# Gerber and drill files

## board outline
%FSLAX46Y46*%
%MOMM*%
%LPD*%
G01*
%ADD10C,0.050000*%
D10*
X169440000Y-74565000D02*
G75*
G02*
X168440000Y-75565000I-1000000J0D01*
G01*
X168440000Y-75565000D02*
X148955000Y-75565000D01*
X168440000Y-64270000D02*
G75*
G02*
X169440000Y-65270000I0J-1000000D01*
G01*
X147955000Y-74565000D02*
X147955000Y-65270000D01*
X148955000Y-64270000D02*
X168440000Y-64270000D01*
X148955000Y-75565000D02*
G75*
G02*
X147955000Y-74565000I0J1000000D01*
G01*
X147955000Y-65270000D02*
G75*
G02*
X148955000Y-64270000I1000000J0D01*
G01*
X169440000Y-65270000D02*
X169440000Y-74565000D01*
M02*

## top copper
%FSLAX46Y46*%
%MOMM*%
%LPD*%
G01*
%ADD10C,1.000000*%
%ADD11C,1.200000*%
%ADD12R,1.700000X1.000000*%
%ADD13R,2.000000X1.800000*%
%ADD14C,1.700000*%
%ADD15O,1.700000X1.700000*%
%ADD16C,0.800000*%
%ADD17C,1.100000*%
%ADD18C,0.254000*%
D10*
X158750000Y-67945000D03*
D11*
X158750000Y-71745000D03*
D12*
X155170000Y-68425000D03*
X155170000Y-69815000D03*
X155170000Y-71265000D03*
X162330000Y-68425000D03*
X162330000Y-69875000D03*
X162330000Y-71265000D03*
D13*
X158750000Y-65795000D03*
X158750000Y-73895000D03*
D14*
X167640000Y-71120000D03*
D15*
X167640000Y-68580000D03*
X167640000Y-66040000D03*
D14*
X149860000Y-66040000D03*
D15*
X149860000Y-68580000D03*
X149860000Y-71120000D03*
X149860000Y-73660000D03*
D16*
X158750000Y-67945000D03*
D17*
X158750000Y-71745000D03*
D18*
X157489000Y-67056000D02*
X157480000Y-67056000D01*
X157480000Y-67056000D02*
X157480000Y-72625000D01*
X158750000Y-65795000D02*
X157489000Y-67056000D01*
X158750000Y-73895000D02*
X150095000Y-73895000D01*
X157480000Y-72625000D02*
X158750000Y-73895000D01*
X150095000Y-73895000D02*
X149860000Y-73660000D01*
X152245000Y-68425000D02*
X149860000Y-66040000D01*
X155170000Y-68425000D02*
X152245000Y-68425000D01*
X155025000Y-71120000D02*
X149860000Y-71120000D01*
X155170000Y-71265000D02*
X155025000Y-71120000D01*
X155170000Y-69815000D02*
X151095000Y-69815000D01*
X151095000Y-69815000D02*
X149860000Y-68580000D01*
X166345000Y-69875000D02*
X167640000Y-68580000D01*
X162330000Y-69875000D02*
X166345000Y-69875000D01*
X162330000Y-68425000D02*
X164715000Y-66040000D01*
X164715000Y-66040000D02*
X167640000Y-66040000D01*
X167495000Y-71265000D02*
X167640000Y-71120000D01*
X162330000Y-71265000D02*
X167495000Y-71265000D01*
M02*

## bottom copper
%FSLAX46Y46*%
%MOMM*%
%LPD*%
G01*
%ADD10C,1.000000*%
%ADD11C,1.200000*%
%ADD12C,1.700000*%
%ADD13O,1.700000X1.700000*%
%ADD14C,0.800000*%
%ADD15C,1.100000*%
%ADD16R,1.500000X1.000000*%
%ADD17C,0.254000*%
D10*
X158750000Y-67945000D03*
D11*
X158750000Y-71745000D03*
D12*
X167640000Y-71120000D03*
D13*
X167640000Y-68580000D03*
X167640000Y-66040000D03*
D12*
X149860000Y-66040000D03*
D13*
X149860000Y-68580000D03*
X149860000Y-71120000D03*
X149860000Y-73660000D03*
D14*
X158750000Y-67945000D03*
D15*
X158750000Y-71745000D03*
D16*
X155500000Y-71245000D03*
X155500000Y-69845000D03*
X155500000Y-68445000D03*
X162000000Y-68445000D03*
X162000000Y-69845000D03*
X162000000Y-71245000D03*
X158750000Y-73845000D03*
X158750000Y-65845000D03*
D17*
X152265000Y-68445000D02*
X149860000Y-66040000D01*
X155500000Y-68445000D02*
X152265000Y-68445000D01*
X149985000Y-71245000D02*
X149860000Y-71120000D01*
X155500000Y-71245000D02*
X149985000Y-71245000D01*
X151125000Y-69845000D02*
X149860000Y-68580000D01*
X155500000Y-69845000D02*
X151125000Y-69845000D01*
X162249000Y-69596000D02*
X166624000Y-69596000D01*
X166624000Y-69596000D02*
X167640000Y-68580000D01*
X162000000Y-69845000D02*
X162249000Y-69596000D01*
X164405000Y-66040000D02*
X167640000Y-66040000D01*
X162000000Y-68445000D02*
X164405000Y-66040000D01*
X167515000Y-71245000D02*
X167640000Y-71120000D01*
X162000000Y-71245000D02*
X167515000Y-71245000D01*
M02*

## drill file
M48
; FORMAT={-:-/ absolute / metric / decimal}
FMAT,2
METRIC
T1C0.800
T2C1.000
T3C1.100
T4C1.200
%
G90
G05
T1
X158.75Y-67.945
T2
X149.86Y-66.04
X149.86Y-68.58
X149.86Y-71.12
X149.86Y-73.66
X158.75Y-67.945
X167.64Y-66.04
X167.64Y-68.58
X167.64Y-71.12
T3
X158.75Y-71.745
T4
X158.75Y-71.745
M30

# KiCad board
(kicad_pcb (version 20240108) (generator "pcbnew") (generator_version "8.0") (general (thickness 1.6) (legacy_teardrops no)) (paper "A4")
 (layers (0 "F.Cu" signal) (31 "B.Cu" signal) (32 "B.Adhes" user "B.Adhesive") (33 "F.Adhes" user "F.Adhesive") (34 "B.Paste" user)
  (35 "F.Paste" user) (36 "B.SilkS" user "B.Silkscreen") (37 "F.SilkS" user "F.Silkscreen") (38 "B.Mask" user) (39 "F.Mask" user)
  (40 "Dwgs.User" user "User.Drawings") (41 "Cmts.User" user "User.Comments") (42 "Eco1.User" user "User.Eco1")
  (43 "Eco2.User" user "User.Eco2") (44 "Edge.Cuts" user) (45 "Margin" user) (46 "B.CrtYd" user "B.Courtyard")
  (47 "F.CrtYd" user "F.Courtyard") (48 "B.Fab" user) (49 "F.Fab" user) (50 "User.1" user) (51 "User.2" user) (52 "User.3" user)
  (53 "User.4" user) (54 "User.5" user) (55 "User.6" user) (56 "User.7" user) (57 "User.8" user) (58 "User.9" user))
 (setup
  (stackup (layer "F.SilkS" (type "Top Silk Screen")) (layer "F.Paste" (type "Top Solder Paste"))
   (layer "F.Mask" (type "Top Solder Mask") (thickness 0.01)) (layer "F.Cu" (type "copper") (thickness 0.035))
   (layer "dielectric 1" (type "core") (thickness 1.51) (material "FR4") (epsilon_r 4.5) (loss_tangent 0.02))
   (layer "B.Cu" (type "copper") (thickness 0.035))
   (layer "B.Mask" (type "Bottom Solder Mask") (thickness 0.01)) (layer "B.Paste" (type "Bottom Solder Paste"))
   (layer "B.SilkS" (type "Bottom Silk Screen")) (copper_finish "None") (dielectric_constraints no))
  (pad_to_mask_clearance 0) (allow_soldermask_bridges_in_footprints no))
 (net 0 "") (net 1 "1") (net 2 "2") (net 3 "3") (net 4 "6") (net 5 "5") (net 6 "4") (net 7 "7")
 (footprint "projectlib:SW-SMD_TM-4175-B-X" (layer "F.Cu") (at 158.75 69.845)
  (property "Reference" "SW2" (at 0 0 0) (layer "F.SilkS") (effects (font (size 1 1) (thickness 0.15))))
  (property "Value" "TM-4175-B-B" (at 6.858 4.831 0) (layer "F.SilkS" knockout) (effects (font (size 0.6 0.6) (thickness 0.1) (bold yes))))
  (pad "" thru_hole circle (at 0 -1.9) (size 1 1) (drill 1) (layers "*.Cu" "*.Mask") (remove_unused_layers no))
  (pad "" thru_hole circle (at 0 1.9) (size 1.2 1.2) (drill 1.2) (layers "*.Cu" "*.Mask") (remove_unused_layers no))
  (pad "1" smd rect (at -3.58 -1.42) (size 1.7 1) (layers "F.Cu" "F.Paste" "F.Mask") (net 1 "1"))
  (pad "2" smd rect (at -3.58 -0.03) (size 1.7 1) (layers "F.Cu" "F.Paste" "F.Mask") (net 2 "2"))
  (pad "3" smd rect (at -3.58 1.42) (size 1.7 1) (layers "F.Cu" "F.Paste" "F.Mask") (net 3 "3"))
  (pad "4" smd rect (at 3.58 -1.42) (size 1.7 1) (layers "F.Cu" "F.Paste" "F.Mask") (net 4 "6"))
  (pad "5" smd rect (at 3.58 0.03) (size 1.7 1) (layers "F.Cu" "F.Paste" "F.Mask") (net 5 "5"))
  (pad "6" smd rect (at 3.58 1.42) (size 1.7 1) (layers "F.Cu" "F.Paste" "F.Mask") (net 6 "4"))
  (pad "7" smd rect (at 0 -4.05) (size 2 1.8) (layers "F.Cu" "F.Paste" "F.Mask") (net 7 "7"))
  (pad "7" smd rect (at 0 4.05) (size 2 1.8) (layers "F.Cu" "F.Paste" "F.Mask") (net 7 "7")))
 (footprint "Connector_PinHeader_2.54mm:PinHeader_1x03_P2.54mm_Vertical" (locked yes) (layer "F.Cu") (at 167.64 71.12 180)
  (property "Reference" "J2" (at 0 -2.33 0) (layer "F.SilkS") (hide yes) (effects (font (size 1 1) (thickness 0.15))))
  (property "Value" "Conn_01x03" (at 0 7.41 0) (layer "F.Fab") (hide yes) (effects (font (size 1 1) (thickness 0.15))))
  (pad "1" thru_hole circle (at 0 0 180) (size 1.7 1.7) (drill 1) (layers "*.Cu" "*.Mask") (remove_unused_layers no) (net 6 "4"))
  (pad "2" thru_hole oval (at 0 2.54 180) (size 1.7 1.7) (drill 1) (layers "*.Cu" "*.Mask") (remove_unused_layers no) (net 5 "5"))
  (pad "3" thru_hole oval (at 0 5.08 180) (size 1.7 1.7) (drill 1) (layers "*.Cu" "*.Mask") (remove_unused_layers no) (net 4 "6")))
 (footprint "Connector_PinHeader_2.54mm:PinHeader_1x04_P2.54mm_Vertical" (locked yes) (layer "F.Cu") (at 149.86 66.04)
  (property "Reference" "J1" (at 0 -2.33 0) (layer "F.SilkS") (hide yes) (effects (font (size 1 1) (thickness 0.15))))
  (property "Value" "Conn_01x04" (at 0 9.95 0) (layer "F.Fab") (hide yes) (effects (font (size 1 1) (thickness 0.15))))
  (pad "1" thru_hole circle (at 0 0) (size 1.7 1.7) (drill 1) (layers "*.Cu" "*.Mask") (remove_unused_layers no) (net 1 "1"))
  (pad "2" thru_hole oval (at 0 2.54) (size 1.7 1.7) (drill 1) (layers "*.Cu" "*.Mask") (remove_unused_layers no) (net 2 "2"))
  (pad "3" thru_hole oval (at 0 5.08) (size 1.7 1.7) (drill 1) (layers "*.Cu" "*.Mask") (remove_unused_layers no) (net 3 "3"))
  (pad "4" thru_hole oval (at 0 7.62) (size 1.7 1.7) (drill 1) (layers "*.Cu" "*.Mask") (remove_unused_layers no) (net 7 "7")))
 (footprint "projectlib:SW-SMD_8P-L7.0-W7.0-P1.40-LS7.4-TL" (layer "B.Cu") (at 158.75 69.845)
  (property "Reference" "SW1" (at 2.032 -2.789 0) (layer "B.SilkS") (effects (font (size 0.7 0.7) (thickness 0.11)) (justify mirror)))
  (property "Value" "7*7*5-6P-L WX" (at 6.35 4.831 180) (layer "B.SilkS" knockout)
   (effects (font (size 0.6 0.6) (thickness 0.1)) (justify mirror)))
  (pad "" thru_hole circle (at 0 -1.9) (size 0.8 0.8) (drill 0.8) (layers "*.Cu" "*.Mask") (remove_unused_layers no))
  (pad "" thru_hole circle (at 0 1.9) (size 1.1 1.1) (drill 1.1) (layers "*.Cu" "*.Mask") (remove_unused_layers no))
  (pad "1" smd rect (at -3.25 1.4) (size 1.5 1) (layers "B.Cu" "B.Paste" "B.Mask") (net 3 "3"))
  (pad "2" smd rect (at -3.25 0) (size 1.5 1) (layers "B.Cu" "B.Paste" "B.Mask") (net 2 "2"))
  (pad "3" smd rect (at -3.25 -1.4) (size 1.5 1) (layers "B.Cu" "B.Paste" "B.Mask") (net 1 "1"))
  (pad "4" smd rect (at 3.25 -1.4) (size 1.5 1) (layers "B.Cu" "B.Paste" "B.Mask") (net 4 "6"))
  (pad "5" smd rect (at 3.25 0) (size 1.5 1) (layers "B.Cu" "B.Paste" "B.Mask") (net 5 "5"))
  (pad "6" smd rect (at 3.25 1.4) (size 1.5 1) (layers "B.Cu" "B.Paste" "B.Mask") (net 6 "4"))
  (pad "7" smd rect (at 0 4) (size 1.5 1) (layers "B.Cu" "B.Paste" "B.Mask"))
  (pad "8" smd rect (at 0 -4) (size 1.5 1) (layers "B.Cu" "B.Paste" "B.Mask")))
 (gr_arc (start 169.44 74.565) (mid 169.147107 75.272107) (end 168.44 75.565) (stroke (width 0.05) (type default)) (layer "Edge.Cuts"))
 (gr_line (start 168.44 75.565) (end 148.955 75.565) (stroke (width 0.05) (type default)) (layer "Edge.Cuts"))
 (gr_arc (start 168.44 64.27) (mid 169.147107 64.562893) (end 169.44 65.27) (stroke (width 0.05) (type default)) (layer "Edge.Cuts"))
 (gr_line (start 147.955 74.565) (end 147.955 65.27) (stroke (width 0.05) (type default)) (layer "Edge.Cuts"))
 (gr_line (start 148.955 64.27) (end 168.44 64.27) (stroke (width 0.05) (type default)) (layer "Edge.Cuts"))
 (gr_arc (start 148.955 75.565) (mid 148.247893 75.272107) (end 147.955 74.565) (stroke (width 0.05) (type default)) (layer "Edge.Cuts"))
 (gr_arc (start 147.955 65.27) (mid 148.247893 64.562893) (end 148.955 64.27) (stroke (width 0.05) (type default)) (layer "Edge.Cuts"))
 (gr_line (start 169.44 65.27) (end 169.44 74.565) (stroke (width 0.05) (type default)) (layer "Edge.Cuts"))
 (segment (start 157.489 67.056) (end 157.48 67.056) (width 0.254) (layer "F.Cu") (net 7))
 (segment (start 157.48 67.056) (end 157.48 72.625) (width 0.254) (layer "F.Cu") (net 7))
 (segment (start 158.75 65.795) (end 157.489 67.056) (width 0.254) (layer "F.Cu") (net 7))
 (segment (start 158.75 73.895) (end 150.095 73.895) (width 0.254) (layer "F.Cu") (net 7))
 (segment (start 157.48 72.625) (end 158.75 73.895) (width 0.254) (layer "F.Cu") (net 7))
 (segment (start 150.095 73.895) (end 149.86 73.66) (width 0.254) (layer "F.Cu") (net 7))
 (segment (start 152.245 68.425) (end 149.86 66.04) (width 0.254) (layer "F.Cu") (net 1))
 (segment (start 155.17 68.425) (end 152.245 68.425) (width 0.254) (layer "F.Cu") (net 1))
 (segment (start 152.265 68.445) (end 149.86 66.04) (width 0.254) (layer "B.Cu") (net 1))
 (segment (start 155.5 68.445) (end 152.265 68.445) (width 0.254) (layer "B.Cu") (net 1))
 (segment (start 155.025 71.12) (end 149.86 71.12) (width 0.254) (layer "F.Cu") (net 3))
 (segment (start 155.17 71.265) (end 155.025 71.12) (width 0.254) (layer "F.Cu") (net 3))
 (segment (start 149.985 71.245) (end 149.86 71.12) (width 0.254) (layer "B.Cu") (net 3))
 (segment (start 155.5 71.245) (end 149.985 71.245) (width 0.254) (layer "B.Cu") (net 3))
 (segment (start 155.17 69.815) (end 151.095 69.815) (width 0.254) (layer "F.Cu") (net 2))
 (segment (start 151.095 69.815) (end 149.86 68.58) (width 0.254) (layer "F.Cu") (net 2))
 (segment (start 151.125 69.845) (end 149.86 68.58) (width 0.254) (layer "B.Cu") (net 2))
 (segment (start 155.5 69.845) (end 151.125 69.845) (width 0.254) (layer "B.Cu") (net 2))
 (segment (start 166.345 69.875) (end 167.64 68.58) (width 0.254) (layer "F.Cu") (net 5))
 (segment (start 162.33 69.875) (end 166.345 69.875) (width 0.254) (layer "F.Cu") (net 5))
 (segment (start 162.249 69.596) (end 166.624 69.596) (width 0.254) (layer "B.Cu") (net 5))
 (segment (start 166.624 69.596) (end 167.64 68.58) (width 0.254) (layer "B.Cu") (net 5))
 (segment (start 162 69.845) (end 162.249 69.596) (width 0.254) (layer "B.Cu") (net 5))
 (segment (start 162.33 68.425) (end 164.715 66.04) (width 0.254) (layer "F.Cu") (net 4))
 (segment (start 164.715 66.04) (end 167.64 66.04) (width 0.254) (layer "F.Cu") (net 4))
 (segment (start 164.405 66.04) (end 167.64 66.04) (width 0.254) (layer "B.Cu") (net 4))
 (segment (start 162 68.445) (end 164.405 66.04) (width 0.254) (layer "B.Cu") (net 4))
 (segment (start 167.495 71.265) (end 167.64 71.12) (width 0.254) (layer "F.Cu") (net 6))
 (segment (start 162.33 71.265) (end 167.495 71.265) (width 0.254) (layer "F.Cu") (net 6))
 (segment (start 167.515 71.245) (end 167.64 71.12) (width 0.254) (layer "B.Cu") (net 6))
 (segment (start 162 71.245) (end 167.515 71.245) (width 0.254) (layer "B.Cu") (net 6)))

